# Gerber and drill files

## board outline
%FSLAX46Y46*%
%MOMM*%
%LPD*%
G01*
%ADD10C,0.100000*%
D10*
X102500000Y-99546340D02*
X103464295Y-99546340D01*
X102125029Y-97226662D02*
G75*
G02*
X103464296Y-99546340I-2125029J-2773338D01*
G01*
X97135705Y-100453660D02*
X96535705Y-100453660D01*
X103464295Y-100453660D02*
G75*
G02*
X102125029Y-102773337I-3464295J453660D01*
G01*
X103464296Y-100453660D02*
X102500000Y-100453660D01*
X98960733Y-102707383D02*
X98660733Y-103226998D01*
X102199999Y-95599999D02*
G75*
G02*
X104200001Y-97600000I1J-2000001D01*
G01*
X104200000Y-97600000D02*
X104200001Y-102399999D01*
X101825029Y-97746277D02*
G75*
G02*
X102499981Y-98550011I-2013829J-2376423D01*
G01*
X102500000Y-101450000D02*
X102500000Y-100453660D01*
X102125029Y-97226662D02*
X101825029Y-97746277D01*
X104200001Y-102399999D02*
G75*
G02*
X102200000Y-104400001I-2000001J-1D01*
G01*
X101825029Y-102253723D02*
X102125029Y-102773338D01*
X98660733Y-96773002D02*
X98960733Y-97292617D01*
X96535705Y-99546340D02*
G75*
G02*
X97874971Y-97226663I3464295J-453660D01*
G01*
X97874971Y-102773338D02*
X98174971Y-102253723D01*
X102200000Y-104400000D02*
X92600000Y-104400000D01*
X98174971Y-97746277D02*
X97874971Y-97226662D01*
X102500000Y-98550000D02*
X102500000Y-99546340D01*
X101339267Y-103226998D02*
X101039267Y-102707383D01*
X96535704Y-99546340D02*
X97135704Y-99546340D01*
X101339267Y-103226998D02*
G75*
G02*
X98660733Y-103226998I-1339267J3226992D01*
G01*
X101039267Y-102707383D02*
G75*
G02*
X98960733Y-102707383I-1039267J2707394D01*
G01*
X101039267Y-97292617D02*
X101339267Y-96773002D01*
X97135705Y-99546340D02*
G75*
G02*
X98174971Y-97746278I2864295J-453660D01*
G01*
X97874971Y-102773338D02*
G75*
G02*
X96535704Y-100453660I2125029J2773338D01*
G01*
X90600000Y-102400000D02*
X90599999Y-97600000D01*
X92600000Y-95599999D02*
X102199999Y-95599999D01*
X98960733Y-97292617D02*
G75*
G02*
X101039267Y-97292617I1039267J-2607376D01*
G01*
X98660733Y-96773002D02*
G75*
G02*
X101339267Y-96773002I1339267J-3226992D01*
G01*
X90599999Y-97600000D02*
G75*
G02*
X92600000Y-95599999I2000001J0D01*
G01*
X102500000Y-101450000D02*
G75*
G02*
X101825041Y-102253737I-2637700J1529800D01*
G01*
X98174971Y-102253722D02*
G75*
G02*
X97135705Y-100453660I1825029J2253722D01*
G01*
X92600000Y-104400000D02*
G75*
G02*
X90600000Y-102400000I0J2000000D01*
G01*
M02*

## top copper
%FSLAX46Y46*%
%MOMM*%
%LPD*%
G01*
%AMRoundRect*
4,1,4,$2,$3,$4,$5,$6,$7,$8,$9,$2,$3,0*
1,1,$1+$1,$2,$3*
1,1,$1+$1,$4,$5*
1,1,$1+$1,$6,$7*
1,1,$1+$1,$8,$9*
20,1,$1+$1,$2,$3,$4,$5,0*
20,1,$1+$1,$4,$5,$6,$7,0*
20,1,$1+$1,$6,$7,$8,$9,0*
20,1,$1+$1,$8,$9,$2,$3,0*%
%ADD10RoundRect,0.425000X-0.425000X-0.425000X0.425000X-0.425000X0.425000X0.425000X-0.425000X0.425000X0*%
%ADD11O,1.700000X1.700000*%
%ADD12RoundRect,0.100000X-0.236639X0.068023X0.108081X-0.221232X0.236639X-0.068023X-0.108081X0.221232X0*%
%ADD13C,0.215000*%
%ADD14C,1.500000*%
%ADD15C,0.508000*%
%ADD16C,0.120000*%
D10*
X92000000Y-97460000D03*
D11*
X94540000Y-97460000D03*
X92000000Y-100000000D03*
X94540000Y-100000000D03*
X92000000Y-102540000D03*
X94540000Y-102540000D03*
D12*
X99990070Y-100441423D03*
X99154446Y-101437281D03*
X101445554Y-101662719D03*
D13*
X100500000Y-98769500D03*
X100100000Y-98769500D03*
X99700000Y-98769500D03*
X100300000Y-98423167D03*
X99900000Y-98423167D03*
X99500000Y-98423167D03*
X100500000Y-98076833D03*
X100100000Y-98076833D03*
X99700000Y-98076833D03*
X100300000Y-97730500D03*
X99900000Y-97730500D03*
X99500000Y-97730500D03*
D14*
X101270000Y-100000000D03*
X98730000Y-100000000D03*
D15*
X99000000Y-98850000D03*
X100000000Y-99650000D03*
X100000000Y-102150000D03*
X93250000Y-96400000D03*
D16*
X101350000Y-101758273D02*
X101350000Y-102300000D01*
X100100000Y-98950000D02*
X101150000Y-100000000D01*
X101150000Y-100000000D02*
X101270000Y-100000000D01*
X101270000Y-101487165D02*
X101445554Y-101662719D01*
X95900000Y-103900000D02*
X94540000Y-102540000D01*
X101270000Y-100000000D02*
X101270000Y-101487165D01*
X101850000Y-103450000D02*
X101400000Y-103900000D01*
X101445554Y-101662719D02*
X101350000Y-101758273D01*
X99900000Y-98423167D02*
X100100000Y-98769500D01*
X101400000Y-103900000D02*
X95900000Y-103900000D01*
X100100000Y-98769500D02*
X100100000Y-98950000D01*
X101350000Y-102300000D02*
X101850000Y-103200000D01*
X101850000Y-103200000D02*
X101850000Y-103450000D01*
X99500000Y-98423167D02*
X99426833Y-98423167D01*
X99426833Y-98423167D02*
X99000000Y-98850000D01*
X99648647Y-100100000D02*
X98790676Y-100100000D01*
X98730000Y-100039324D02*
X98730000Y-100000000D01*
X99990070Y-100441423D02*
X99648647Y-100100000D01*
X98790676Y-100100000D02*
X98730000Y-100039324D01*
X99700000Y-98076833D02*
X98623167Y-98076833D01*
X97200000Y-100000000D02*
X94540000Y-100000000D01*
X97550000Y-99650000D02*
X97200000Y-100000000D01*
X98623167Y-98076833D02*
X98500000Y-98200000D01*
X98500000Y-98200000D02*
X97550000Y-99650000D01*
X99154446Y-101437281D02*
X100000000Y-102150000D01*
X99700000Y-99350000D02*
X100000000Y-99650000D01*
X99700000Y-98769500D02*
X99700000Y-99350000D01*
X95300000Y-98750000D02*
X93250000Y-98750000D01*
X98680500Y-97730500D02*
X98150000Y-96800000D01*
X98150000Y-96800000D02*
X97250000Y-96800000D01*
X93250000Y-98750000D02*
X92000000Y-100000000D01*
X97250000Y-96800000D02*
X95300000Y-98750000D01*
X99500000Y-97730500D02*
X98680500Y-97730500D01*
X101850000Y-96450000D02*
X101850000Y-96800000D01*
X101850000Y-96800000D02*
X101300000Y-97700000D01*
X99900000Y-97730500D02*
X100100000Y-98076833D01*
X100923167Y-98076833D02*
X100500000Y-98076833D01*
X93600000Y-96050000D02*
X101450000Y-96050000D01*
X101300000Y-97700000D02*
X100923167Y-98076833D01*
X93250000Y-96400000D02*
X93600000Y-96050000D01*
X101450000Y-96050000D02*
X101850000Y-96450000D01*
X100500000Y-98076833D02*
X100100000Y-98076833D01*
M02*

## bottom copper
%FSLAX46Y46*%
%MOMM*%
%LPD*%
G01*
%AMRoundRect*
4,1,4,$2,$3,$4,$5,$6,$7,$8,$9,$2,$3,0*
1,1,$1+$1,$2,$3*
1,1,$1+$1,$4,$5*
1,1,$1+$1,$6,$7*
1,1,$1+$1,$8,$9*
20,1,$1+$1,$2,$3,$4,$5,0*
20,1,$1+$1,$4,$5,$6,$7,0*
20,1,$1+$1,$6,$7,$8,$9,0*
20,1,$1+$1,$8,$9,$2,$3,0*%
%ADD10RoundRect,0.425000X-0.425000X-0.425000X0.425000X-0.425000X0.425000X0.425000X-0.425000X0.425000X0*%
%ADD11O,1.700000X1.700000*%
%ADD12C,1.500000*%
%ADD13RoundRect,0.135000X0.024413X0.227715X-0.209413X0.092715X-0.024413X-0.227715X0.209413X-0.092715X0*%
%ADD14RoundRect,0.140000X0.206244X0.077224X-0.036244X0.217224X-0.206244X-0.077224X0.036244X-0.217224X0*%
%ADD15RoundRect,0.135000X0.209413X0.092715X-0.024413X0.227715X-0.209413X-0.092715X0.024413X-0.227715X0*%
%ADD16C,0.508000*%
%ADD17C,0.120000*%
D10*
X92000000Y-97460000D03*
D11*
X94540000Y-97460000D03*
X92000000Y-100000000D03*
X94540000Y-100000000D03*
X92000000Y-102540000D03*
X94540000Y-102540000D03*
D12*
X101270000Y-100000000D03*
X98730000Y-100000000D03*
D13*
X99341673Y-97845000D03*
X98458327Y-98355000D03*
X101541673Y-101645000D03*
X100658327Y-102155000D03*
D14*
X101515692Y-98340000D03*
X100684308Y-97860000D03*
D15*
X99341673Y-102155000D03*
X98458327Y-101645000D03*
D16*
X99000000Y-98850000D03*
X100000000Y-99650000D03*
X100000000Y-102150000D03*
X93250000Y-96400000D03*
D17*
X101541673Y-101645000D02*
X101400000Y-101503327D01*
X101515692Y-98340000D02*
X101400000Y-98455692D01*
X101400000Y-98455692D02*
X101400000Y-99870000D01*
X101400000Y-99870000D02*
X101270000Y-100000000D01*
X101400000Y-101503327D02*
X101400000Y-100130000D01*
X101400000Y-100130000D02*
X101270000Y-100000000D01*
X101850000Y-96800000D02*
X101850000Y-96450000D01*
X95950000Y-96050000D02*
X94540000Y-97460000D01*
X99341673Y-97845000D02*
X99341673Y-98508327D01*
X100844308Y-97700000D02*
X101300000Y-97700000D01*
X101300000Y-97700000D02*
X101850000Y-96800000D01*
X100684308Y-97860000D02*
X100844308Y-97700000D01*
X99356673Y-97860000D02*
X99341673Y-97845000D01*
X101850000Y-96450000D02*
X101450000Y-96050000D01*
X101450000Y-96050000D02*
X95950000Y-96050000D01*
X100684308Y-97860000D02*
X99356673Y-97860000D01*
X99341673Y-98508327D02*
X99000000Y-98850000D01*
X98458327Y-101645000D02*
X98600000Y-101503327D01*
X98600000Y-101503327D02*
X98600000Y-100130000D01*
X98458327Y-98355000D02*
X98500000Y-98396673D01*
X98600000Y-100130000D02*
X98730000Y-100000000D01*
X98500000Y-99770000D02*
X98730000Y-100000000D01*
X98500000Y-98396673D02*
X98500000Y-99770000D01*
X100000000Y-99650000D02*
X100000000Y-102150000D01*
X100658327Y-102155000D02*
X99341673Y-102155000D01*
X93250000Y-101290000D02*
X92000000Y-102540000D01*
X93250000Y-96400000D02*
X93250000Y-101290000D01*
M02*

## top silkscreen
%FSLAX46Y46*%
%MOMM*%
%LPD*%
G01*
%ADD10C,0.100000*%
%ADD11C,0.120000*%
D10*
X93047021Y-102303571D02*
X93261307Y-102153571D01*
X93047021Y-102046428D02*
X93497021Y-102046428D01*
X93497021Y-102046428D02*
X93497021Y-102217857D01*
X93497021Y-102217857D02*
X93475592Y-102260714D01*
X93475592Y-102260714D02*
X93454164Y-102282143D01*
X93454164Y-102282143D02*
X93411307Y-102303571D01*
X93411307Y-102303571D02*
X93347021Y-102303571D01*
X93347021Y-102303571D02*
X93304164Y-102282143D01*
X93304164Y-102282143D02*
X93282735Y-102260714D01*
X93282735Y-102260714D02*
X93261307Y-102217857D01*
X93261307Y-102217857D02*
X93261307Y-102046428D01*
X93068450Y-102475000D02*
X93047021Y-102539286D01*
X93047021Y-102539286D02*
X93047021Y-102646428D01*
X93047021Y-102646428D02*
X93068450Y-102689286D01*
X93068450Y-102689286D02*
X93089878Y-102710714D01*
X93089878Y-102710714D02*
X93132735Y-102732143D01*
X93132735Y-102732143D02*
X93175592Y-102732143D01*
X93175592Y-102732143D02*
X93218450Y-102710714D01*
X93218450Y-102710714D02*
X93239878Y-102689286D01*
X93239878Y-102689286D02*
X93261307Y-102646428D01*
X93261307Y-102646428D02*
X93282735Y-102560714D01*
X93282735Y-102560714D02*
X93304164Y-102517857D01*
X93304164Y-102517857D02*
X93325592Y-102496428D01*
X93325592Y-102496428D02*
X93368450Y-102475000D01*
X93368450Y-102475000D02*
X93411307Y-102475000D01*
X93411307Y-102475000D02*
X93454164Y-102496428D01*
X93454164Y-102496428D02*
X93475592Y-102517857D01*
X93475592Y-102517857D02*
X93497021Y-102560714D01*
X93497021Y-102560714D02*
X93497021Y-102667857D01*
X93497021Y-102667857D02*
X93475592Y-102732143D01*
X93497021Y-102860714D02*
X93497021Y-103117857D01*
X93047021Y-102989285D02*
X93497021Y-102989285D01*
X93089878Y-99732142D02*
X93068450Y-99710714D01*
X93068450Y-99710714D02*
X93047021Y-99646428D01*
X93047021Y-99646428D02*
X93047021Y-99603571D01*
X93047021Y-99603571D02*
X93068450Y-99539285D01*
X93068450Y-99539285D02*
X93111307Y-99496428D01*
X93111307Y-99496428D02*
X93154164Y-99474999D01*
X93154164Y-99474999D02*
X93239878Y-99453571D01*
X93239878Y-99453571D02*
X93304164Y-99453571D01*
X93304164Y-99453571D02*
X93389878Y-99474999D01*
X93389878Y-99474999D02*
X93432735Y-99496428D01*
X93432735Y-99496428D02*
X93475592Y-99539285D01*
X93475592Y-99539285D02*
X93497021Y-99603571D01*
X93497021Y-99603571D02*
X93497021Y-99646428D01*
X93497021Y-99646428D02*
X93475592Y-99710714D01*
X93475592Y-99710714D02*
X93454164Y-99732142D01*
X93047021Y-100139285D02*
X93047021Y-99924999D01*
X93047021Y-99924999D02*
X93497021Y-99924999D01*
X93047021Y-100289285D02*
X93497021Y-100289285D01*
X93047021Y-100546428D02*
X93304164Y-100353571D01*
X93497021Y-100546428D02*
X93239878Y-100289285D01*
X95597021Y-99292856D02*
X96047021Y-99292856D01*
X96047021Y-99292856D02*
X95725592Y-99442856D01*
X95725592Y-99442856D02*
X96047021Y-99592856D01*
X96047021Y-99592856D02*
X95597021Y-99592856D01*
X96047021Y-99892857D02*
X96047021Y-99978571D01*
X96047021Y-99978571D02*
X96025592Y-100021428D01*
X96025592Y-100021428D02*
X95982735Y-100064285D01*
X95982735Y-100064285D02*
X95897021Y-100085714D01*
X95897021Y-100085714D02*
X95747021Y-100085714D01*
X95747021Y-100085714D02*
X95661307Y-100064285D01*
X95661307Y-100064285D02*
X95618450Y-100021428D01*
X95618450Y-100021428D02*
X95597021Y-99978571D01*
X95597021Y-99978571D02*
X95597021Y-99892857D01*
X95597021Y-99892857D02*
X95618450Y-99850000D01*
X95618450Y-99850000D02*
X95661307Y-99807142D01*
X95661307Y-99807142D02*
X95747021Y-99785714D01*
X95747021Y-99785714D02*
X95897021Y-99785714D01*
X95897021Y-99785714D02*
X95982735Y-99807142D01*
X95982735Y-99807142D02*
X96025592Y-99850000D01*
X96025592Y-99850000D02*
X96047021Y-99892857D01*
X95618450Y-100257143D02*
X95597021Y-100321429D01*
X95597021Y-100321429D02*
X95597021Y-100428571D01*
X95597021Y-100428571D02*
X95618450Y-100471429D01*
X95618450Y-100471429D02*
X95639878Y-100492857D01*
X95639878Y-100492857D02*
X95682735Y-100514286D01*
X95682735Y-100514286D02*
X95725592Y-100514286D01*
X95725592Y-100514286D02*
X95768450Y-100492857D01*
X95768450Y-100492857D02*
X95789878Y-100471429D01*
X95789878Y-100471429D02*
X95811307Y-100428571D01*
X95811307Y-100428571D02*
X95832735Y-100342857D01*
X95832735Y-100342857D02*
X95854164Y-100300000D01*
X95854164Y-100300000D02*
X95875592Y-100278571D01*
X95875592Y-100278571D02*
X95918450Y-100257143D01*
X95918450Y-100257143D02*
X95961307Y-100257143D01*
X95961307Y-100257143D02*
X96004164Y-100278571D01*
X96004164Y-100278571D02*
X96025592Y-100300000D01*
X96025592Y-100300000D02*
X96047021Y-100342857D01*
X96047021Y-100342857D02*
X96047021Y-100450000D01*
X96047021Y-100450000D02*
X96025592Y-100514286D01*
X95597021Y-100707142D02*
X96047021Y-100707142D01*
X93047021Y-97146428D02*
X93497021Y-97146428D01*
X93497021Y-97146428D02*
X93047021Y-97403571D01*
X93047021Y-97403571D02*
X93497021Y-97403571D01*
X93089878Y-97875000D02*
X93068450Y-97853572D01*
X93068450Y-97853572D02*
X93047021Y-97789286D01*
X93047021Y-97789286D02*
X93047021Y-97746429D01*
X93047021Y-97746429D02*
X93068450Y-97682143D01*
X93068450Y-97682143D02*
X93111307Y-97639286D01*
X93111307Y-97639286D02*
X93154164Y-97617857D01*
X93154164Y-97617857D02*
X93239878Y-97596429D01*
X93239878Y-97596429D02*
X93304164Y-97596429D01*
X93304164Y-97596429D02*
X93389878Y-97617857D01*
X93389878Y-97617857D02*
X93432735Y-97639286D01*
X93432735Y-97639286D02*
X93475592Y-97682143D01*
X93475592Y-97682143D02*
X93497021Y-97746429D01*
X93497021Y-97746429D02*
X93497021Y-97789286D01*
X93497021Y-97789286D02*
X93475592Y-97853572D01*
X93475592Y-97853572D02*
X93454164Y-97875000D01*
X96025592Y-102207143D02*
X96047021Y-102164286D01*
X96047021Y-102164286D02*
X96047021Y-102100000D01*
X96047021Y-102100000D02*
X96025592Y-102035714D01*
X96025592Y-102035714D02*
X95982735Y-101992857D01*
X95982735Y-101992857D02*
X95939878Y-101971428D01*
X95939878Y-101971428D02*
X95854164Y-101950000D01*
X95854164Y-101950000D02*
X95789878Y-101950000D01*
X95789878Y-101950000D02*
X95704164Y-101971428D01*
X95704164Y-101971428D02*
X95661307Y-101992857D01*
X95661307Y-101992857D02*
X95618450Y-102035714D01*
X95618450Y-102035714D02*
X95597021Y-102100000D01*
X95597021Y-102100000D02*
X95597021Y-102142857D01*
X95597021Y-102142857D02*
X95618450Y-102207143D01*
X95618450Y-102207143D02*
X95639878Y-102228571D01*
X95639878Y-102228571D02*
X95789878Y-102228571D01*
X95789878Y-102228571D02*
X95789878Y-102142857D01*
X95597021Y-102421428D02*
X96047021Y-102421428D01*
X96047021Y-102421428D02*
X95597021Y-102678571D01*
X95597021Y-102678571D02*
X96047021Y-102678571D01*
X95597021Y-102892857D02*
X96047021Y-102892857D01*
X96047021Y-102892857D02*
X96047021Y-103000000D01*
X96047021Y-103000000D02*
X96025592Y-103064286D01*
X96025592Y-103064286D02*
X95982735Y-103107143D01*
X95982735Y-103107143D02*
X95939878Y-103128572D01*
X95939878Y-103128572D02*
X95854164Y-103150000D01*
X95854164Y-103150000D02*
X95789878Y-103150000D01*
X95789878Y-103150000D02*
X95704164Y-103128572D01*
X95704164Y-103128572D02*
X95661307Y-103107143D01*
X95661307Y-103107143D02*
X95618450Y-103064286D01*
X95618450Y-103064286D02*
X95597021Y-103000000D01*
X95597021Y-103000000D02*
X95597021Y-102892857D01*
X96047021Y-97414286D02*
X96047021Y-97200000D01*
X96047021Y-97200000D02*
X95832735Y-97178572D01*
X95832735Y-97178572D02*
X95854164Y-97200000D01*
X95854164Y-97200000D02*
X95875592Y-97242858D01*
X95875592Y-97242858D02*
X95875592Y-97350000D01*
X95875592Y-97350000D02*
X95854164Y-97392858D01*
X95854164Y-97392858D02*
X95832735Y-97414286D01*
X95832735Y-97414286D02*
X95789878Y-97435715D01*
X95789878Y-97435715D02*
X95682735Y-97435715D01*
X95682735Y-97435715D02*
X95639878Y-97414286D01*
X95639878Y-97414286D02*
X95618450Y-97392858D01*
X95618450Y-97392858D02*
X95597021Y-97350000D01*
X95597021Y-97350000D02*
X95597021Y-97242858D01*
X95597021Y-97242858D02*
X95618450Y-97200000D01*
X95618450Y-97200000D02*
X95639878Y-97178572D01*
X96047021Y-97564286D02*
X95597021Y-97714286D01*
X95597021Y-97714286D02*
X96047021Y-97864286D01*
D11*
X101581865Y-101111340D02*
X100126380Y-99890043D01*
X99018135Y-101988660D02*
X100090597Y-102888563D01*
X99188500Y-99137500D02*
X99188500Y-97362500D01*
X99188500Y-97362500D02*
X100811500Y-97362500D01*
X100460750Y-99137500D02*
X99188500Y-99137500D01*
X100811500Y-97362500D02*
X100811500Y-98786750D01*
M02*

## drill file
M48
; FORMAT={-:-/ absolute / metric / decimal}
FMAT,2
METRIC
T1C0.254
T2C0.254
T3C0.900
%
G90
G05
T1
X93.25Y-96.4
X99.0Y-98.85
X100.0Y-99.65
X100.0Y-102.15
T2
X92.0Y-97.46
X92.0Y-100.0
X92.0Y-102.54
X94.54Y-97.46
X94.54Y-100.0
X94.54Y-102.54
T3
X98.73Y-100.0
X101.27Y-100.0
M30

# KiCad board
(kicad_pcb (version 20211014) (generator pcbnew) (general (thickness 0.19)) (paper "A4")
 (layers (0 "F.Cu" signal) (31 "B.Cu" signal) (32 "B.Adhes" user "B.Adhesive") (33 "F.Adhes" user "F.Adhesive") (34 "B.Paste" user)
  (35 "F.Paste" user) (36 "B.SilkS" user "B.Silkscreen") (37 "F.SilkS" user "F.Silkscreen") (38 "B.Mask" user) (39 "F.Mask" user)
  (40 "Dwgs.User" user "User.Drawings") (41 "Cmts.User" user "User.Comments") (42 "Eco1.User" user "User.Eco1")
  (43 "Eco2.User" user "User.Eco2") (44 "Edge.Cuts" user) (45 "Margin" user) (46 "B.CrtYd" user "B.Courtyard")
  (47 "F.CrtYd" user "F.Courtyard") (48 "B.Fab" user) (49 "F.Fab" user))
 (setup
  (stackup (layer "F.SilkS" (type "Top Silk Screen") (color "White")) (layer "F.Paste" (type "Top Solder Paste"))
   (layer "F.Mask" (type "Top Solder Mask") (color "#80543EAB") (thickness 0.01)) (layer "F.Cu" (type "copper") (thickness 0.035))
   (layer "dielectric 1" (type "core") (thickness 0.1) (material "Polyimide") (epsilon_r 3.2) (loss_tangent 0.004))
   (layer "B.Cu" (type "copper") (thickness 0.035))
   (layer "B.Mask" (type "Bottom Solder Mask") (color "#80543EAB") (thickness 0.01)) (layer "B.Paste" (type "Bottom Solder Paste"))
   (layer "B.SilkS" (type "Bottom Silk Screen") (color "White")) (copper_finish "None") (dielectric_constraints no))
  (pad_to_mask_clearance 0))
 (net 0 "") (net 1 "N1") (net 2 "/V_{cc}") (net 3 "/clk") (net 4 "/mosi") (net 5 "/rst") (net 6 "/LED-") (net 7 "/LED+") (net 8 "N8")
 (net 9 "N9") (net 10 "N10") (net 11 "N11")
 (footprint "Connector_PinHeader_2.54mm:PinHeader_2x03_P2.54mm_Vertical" (layer "F.Cu") (at 92 97.46)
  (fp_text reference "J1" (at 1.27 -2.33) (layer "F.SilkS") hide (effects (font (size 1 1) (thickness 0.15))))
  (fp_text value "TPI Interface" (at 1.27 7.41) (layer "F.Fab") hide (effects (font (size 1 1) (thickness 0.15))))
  (pad "1" thru_hole roundrect (at 0 0) (size 1.7 1.7) (drill 0.254) (layers *.Cu *.Mask) (roundrect_rratio 0.25) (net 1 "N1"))
  (pad "2" thru_hole oval (at 2.54 0) (size 1.7 1.7) (drill 0.254) (layers *.Cu *.Mask) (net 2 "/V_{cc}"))
  (pad "3" thru_hole oval (at 0 2.54) (size 1.7 1.7) (drill 0.254) (layers *.Cu *.Mask) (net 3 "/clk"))
  (pad "4" thru_hole oval (at 2.54 2.54) (size 1.7 1.7) (drill 0.254) (layers *.Cu *.Mask) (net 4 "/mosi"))
  (pad "5" thru_hole oval (at 0 5.08) (size 1.7 1.7) (drill 0.254) (layers *.Cu *.Mask) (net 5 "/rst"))
  (pad "6" thru_hole oval (at 2.54 5.08) (size 1.7 1.7) (drill 0.254) (layers *.Cu *.Mask) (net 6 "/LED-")))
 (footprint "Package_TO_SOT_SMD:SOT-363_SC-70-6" (layer "F.Cu") (at 100.3 101.55 -40)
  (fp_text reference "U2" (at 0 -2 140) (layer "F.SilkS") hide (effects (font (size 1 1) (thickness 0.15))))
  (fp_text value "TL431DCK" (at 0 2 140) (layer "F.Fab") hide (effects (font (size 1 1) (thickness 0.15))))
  (fp_line (start 0.7 -1.16) (end -1.2 -1.16) (layer "F.SilkS") (width 0.12))
  (fp_line (start -0.7 1.16) (end 0.7 1.16) (layer "F.SilkS") (width 0.12))
  (pad "1" smd roundrect (at -0.95 -0.65 320) (size 0.65 0.4) (layers "F.Cu" "F.Paste" "F.Mask") (roundrect_rratio 0.25) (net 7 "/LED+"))
  (pad "3" smd roundrect (at -0.95 0.65 320) (size 0.65 0.4) (layers "F.Cu" "F.Paste" "F.Mask") (roundrect_rratio 0.25) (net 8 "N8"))
  (pad "6" smd roundrect (at 0.95 -0.65 320) (size 0.65 0.4) (layers "F.Cu" "F.Paste" "F.Mask") (roundrect_rratio 0.25) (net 6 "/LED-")))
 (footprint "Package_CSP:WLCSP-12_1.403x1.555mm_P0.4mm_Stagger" (layer "F.Cu") (at 100 98.25 180) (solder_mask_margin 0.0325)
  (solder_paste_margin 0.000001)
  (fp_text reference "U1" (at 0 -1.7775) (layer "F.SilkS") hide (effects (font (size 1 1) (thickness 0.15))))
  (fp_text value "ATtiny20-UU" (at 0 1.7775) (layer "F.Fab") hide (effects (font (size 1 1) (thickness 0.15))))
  (fp_line (start 0.8115 -0.8875) (end 0.8115 0.8875) (layer "F.SilkS") (width 0.12))
  (fp_line (start 0.8115 0.8875) (end -0.8115 0.8875) (layer "F.SilkS") (width 0.12))
  (fp_line (start -0.46075 -0.8875) (end 0.8115 -0.8875) (layer "F.SilkS") (width 0.12))
  (fp_line (start -0.8115 0.8875) (end -0.8115 -0.53675) (layer "F.SilkS") (width 0.12))
  (pad "A1" smd circle locked (at -0.5 -0.5195 180) (size 0.215 0.215) (layers "F.Cu" "F.Paste" "F.Mask") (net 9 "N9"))
  (pad "A3" smd circle locked (at -0.1 -0.5195 180) (size 0.215 0.215) (layers "F.Cu" "F.Paste" "F.Mask") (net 6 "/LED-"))
  (pad "A5" smd circle locked (at 0.3 -0.5195 180) (size 0.215 0.215) (layers "F.Cu" "F.Paste" "F.Mask") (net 8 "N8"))
  (pad "B2" smd circle locked (at -0.3 -0.173167 180) (size 0.215 0.215) (layers "F.Cu" "F.Paste" "F.Mask") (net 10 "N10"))
  (pad "B4" smd circle locked (at 0.1 -0.173167 180) (size 0.215 0.215) (layers "F.Cu" "F.Paste" "F.Mask") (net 6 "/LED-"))
  (pad "B6" smd circle locked (at 0.5 -0.173167 180) (size 0.215 0.215) (layers "F.Cu" "F.Paste" "F.Mask") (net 2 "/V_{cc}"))
  (pad "C1" smd circle locked (at -0.5 0.173167 180) (size 0.215 0.215) (layers "F.Cu" "F.Paste" "F.Mask") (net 5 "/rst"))
  (pad "C3" smd circle locked (at -0.1 0.173167 180) (size 0.215 0.215) (layers "F.Cu" "F.Paste" "F.Mask") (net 5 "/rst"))
  (pad "C5" smd circle locked (at 0.3 0.173167 180) (size 0.215 0.215) (layers "F.Cu" "F.Paste" "F.Mask") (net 4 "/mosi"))
  (pad "D2" smd circle locked (at -0.3 0.5195 180) (size 0.215 0.215) (layers "F.Cu" "F.Paste" "F.Mask") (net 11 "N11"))
  (pad "D4" smd circle locked (at 0.1 0.5195 180) (size 0.215 0.215) (layers "F.Cu" "F.Paste" "F.Mask") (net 5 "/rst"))
  (pad "D6" smd circle locked (at 0.5 0.5195 180) (size 0.215 0.215) (layers "F.Cu" "F.Paste" "F.Mask") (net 3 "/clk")))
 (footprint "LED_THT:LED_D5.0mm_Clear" (layer "B.Cu") (at 100 100 180)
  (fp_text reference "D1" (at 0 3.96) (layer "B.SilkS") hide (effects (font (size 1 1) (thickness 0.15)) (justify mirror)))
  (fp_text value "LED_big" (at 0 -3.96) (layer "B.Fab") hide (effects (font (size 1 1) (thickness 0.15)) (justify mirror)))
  (pad "1" thru_hole circle (at -1.27 0 180) (size 1.5 1.5) (drill 0.9) (layers *.Cu *.Mask) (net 6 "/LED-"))
  (pad "2" thru_hole circle (at 1.27 0 180) (size 1.5 1.5) (drill 0.9) (layers *.Cu *.Mask) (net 7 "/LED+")))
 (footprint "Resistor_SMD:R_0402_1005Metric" (layer "B.Cu") (at 98.9 98.1 -150)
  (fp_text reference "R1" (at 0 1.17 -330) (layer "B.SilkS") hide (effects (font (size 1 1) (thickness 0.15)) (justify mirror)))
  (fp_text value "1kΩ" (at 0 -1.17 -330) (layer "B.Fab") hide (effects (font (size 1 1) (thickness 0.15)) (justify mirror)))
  (pad "1" smd roundrect locked (at -0.51 0 210) (size 0.54 0.64) (layers "B.Cu" "B.Paste" "B.Mask") (roundrect_rratio 0.25)
   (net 2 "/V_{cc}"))
  (pad "2" smd roundrect locked (at 0.51 0 210) (size 0.54 0.64) (layers "B.Cu" "B.Paste" "B.Mask") (roundrect_rratio 0.25) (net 7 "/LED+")))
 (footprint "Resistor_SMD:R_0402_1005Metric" (layer "B.Cu") (at 101.1 101.9 -150)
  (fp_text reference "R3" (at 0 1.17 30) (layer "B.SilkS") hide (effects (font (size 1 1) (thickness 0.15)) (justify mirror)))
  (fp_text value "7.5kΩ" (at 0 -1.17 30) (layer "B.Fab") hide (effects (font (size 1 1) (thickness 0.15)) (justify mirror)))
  (pad "1" smd roundrect locked (at -0.51 0 210) (size 0.54 0.64) (layers "B.Cu" "B.Paste" "B.Mask") (roundrect_rratio 0.25) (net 6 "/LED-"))
  (pad "2" smd roundrect locked (at 0.51 0 210) (size 0.54 0.64) (layers "B.Cu" "B.Paste" "B.Mask") (roundrect_rratio 0.25) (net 8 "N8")))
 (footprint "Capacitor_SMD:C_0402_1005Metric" (layer "B.Cu") (at 101.1 98.1 150)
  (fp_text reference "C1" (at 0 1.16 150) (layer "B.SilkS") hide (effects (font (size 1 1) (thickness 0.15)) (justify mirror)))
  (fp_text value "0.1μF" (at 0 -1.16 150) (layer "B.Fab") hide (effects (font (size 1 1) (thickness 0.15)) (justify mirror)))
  (pad "1" smd roundrect locked (at -0.48 0 150) (size 0.56 0.62) (layers "B.Cu" "B.Paste" "B.Mask") (roundrect_rratio 0.25) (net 6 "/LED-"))
  (pad "2" smd roundrect locked (at 0.48 0 150) (size 0.56 0.62) (layers "B.Cu" "B.Paste" "B.Mask") (roundrect_rratio 0.25)
   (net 2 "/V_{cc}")))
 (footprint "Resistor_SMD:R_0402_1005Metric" (layer "B.Cu") (at 98.9 101.9 150)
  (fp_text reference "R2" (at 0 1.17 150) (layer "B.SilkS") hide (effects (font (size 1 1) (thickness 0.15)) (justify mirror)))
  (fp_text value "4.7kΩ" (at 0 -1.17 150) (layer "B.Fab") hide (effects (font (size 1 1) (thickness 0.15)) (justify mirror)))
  (pad "1" smd roundrect locked (at -0.51 0 150) (size 0.54 0.64) (layers "B.Cu" "B.Paste" "B.Mask") (roundrect_rratio 0.25) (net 8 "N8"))
  (pad "2" smd roundrect locked (at 0.51 0 150) (size 0.54 0.64) (layers "B.Cu" "B.Paste" "B.Mask") (roundrect_rratio 0.25) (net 7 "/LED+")))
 (gr_line (start 102.5 99.54634) (end 103.464295 99.54634) (layer "Edge.Cuts") (width 0.1))
 (gr_arc (start 102.125029 97.226662) (mid 103.025783 98.253063) (end 103.464295 99.54634) (layer "Edge.Cuts") (width 0.1))
 (gr_line (start 97.135705 100.45366) (end 96.535705 100.45366) (layer "Edge.Cuts") (width 0.1))
 (gr_arc (start 103.464295 100.45366) (mid 103.025783 101.746936) (end 102.125029 102.773338) (layer "Edge.Cuts") (width 0.1))
 (gr_line (start 103.464296 100.45366) (end 102.5 100.45366) (layer "Edge.Cuts") (width 0.1))
 (gr_line (start 98.960733 102.707383) (end 98.660733 103.226998) (layer "Edge.Cuts") (width 0.1))
 (gr_arc (start 102.199999 95.599999) (mid 103.614213 96.185786) (end 104.2 97.6) (layer "Edge.Cuts") (width 0.1))
 (gr_line (start 104.2 97.6) (end 104.200001 102.399999) (layer "Edge.Cuts") (width 0.1))
 (gr_arc (start 101.825029 97.746277) (mid 102.196609 98.119506) (end 102.5 98.55) (layer "Edge.Cuts") (width 0.1))
 (gr_line (start 102.5 101.45) (end 102.5 100.45366) (layer "Edge.Cuts") (width 0.1))
 (gr_line (start 102.125029 97.226662) (end 101.825029 97.746277) (layer "Edge.Cuts") (width 0.1))
 (gr_arc (start 104.200001 102.399999) (mid 103.614214 103.814213) (end 102.2 104.4) (layer "Edge.Cuts") (width 0.1))
 (gr_line (start 101.825029 102.253723) (end 102.125029 102.773338) (layer "Edge.Cuts") (width 0.1))
 (gr_line (start 98.660733 96.773002) (end 98.960733 97.292617) (layer "Edge.Cuts") (width 0.1))
 (gr_arc (start 96.535705 99.54634) (mid 96.974217 98.253064) (end 97.874971 97.226662) (layer "Edge.Cuts") (width 0.1))
 (gr_line (start 97.874971 102.773338) (end 98.174971 102.253723) (layer "Edge.Cuts") (width 0.1))
 (gr_line (start 102.2 104.4) (end 92.6 104.4) (layer "Edge.Cuts") (width 0.1))
 (gr_line (start 98.174971 97.746277) (end 97.874971 97.226662) (layer "Edge.Cuts") (width 0.1))
 (gr_line (start 102.5 98.55) (end 102.5 99.54634) (layer "Edge.Cuts") (width 0.1))
 (gr_line (start 101.339267 103.226998) (end 101.039267 102.707383) (layer "Edge.Cuts") (width 0.1))
 (gr_line (start 96.535704 99.54634) (end 97.135704 99.54634) (layer "Edge.Cuts") (width 0.1))
 (gr_arc (start 101.339267 103.226998) (mid 100 103.493874) (end 98.660733 103.226998) (layer "Edge.Cuts") (width 0.1))
 (gr_arc (start 101.039267 102.707383) (mid 100 102.899999) (end 98.960733 102.707383) (layer "Edge.Cuts") (width 0.1))
 (gr_line (start 101.039267 97.292617) (end 101.339267 96.773002) (layer "Edge.Cuts") (width 0.1))
 (gr_arc (start 97.135705 99.54634) (mid 97.488527 98.550001) (end 98.174971 97.746278) (layer "Edge.Cuts") (width 0.1))
 (gr_arc (start 97.874971 102.773338) (mid 96.974217 101.746937) (end 96.535705 100.45366) (layer "Edge.Cuts") (width 0.1))
 (gr_line (start 90.6 102.4) (end 90.599999 97.6) (layer "Edge.Cuts") (width 0.1))
 (gr_line (start 92.6 95.599999) (end 102.199999 95.599999) (layer "Edge.Cuts") (width 0.1))
 (gr_arc (start 98.960733 97.292617) (mid 100 97.093129) (end 101.039267 97.292617) (layer "Edge.Cuts") (width 0.1))
 (gr_arc (start 98.660733 96.773002) (mid 100 96.506126) (end 101.339267 96.773002) (layer "Edge.Cuts") (width 0.1))
 (gr_arc (start 90.599999 97.6) (mid 91.185786 96.185786) (end 92.6 95.599999) (layer "Edge.Cuts") (width 0.1))
 (gr_arc (start 102.5 101.45) (mid 102.197355 101.881121) (end 101.825029 102.253723) (layer "Edge.Cuts") (width 0.1))
 (gr_arc (start 98.174971 102.253722) (mid 97.488527 101.449999) (end 97.135705 100.45366) (layer "Edge.Cuts") (width 0.1))
 (gr_arc (start 92.6 104.4) (mid 91.185786 103.814214) (end 90.6 102.4) (layer "Edge.Cuts") (width 0.1))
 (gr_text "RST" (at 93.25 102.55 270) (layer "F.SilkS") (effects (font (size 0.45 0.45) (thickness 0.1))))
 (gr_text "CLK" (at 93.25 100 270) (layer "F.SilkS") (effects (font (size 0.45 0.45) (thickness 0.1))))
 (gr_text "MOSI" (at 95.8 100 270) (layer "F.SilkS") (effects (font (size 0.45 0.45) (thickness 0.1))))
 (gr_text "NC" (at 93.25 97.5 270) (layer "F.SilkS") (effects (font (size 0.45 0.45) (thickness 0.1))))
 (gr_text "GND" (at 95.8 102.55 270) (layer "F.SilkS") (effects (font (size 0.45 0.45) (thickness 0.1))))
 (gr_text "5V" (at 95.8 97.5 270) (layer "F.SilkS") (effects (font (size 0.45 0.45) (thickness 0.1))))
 (segment (start 101.35 101.758273) (end 101.35 102.3) (width 0.12) (layer "F.Cu") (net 6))
 (segment (start 100.1 98.95) (end 101.15 100) (width 0.12) (layer "F.Cu") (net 6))
 (segment (start 101.15 100) (end 101.27 100) (width 0.12) (layer "F.Cu") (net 6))
 (segment (start 101.27 101.487165) (end 101.445554 101.662719) (width 0.12) (layer "F.Cu") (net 6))
 (segment (start 95.9 103.9) (end 94.54 102.54) (width 0.12) (layer "F.Cu") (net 6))
 (segment (start 101.27 100) (end 101.27 101.487165) (width 0.12) (layer "F.Cu") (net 6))
 (segment (start 101.85 103.45) (end 101.4 103.9) (width 0.12) (layer "F.Cu") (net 6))
 (segment (start 101.445554 101.662719) (end 101.35 101.758273) (width 0.12) (layer "F.Cu") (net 6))
 (segment (start 99.9 98.423167) (end 100.1 98.7695) (width 0.12) (layer "F.Cu") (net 6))
 (segment (start 101.4 103.9) (end 95.9 103.9) (width 0.12) (layer "F.Cu") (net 6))
 (segment (start 100.1 98.7695) (end 100.1 98.95) (width 0.12) (layer "F.Cu") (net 6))
 (segment (start 101.35 102.3) (end 101.85 103.2) (width 0.12) (layer "F.Cu") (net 6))
 (segment (start 101.85 103.2) (end 101.85 103.45) (width 0.12) (layer "F.Cu") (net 6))
 (segment (start 101.541673 101.645) (end 101.4 101.503327) (width 0.12) (layer "B.Cu") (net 6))
 (segment (start 101.515692 98.34) (end 101.4 98.455692) (width 0.12) (layer "B.Cu") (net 6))
 (segment (start 101.4 98.455692) (end 101.4 99.87) (width 0.12) (layer "B.Cu") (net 6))
 (segment (start 101.4 99.87) (end 101.27 100) (width 0.12) (layer "B.Cu") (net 6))
 (segment (start 101.4 101.503327) (end 101.4 100.13) (width 0.12) (layer "B.Cu") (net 6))
 (segment (start 101.4 100.13) (end 101.27 100) (width 0.12) (layer "B.Cu") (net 6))
 (segment (start 99.5 98.423167) (end 99.426833 98.423167) (width 0.12) (layer "F.Cu") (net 2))
 (segment (start 99.426833 98.423167) (end 99 98.85) (width 0.12) (layer "F.Cu") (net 2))
 (via (at 99 98.85) (size 0.508) (drill 0.254) (layers "F.Cu" "B.Cu") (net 2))
 (segment (start 101.85 96.8) (end 101.85 96.45) (width 0.12) (layer "B.Cu") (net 2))
 (segment (start 95.95 96.05) (end 94.54 97.46) (width 0.12) (layer "B.Cu") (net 2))
 (segment (start 99.341673 97.845) (end 99.341673 98.508327) (width 0.12) (layer "B.Cu") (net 2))
 (segment (start 100.844308 97.7) (end 101.3 97.7) (width 0.12) (layer "B.Cu") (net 2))
 (segment (start 101.3 97.7) (end 101.85 96.8) (width 0.12) (layer "B.Cu") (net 2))
 (segment (start 100.684308 97.86) (end 100.844308 97.7) (width 0.12) (layer "B.Cu") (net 2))
 (segment (start 99.356673 97.86) (end 99.341673 97.845) (width 0.12) (layer "B.Cu") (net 2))
 (segment (start 101.85 96.45) (end 101.45 96.05) (width 0.12) (layer "B.Cu") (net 2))
 (segment (start 101.45 96.05) (end 95.95 96.05) (width 0.12) (layer "B.Cu") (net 2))
 (segment (start 100.684308 97.86) (end 99.356673 97.86) (width 0.12) (layer "B.Cu") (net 2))
 (segment (start 99.341673 98.508327) (end 99 98.85) (width 0.12) (layer "B.Cu") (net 2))
 (segment (start 99.648647 100.1) (end 98.790676 100.1) (width 0.12) (layer "F.Cu") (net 7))
 (segment (start 98.73 100.039324) (end 98.73 100) (width 0.12) (layer "F.Cu") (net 7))
 (segment (start 99.99007 100.441423) (end 99.648647 100.1) (width 0.12) (layer "F.Cu") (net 7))
 (segment (start 98.790676 100.1) (end 98.73 100.039324) (width 0.12) (layer "F.Cu") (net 7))
 (segment (start 98.458327 101.645) (end 98.6 101.503327) (width 0.12) (layer "B.Cu") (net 7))
 (segment (start 98.6 101.503327) (end 98.6 100.13) (width 0.12) (layer "B.Cu") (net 7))
 (segment (start 98.458327 98.355) (end 98.5 98.396673) (width 0.12) (layer "B.Cu") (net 7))
 (segment (start 98.6 100.13) (end 98.73 100) (width 0.12) (layer "B.Cu") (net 7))
 (segment (start 98.5 99.77) (end 98.73 100) (width 0.12) (layer "B.Cu") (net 7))
 (segment (start 98.5 98.396673) (end 98.5 99.77) (width 0.12) (layer "B.Cu") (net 7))
 (segment (start 99.7 98.076833) (end 98.623167 98.076833) (width 0.12) (layer "F.Cu") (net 4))
 (segment (start 97.2 100) (end 94.54 100) (width 0.12) (layer "F.Cu") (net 4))
 (segment (start 97.55 99.65) (end 97.2 100) (width 0.12) (layer "F.Cu") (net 4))
 (segment (start 98.623167 98.076833) (end 98.5 98.2) (width 0.12) (layer "F.Cu") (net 4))
 (segment (start 98.5 98.2) (end 97.55 99.65) (width 0.12) (layer "F.Cu") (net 4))
 (segment (start 99.154446 101.437281) (end 100 102.15) (width 0.12) (layer "F.Cu") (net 8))
 (segment (start 99.7 99.35) (end 100 99.65) (width 0.12) (layer "F.Cu") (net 8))
 (segment (start 99.7 98.7695) (end 99.7 99.35) (width 0.12) (layer "F.Cu") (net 8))
 (via (at 100 99.65) (size 0.508) (drill 0.254) (layers "F.Cu" "B.Cu") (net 8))
 (via (at 100 102.15) (size 0.508) (drill 0.254) (layers "F.Cu" "B.Cu") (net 8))
 (segment (start 100 99.65) (end 100 102.15) (width 0.12) (layer "B.Cu") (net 8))
 (segment (start 100.658327 102.155) (end 99.341673 102.155) (width 0.12) (layer "B.Cu") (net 8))
 (segment (start 95.3 98.75) (end 93.25 98.75) (width 0.12) (layer "F.Cu") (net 3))
 (segment (start 98.6805 97.7305) (end 98.15 96.8) (width 0.12) (layer "F.Cu") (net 3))
 (segment (start 98.15 96.8) (end 97.25 96.8) (width 0.12) (layer "F.Cu") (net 3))
 (segment (start 93.25 98.75) (end 92 100) (width 0.12) (layer "F.Cu") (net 3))
 (segment (start 97.25 96.8) (end 95.3 98.75) (width 0.12) (layer "F.Cu") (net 3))
 (segment (start 99.5 97.7305) (end 98.6805 97.7305) (width 0.12) (layer "F.Cu") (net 3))
 (segment (start 101.85 96.45) (end 101.85 96.8) (width 0.12) (layer "F.Cu") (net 5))
 (segment (start 101.85 96.8) (end 101.3 97.7) (width 0.12) (layer "F.Cu") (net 5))
 (segment (start 99.9 97.7305) (end 100.1 98.076833) (width 0.12) (layer "F.Cu") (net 5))
 (segment (start 100.923167 98.076833) (end 100.5 98.076833) (width 0.12) (layer "F.Cu") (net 5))
 (segment (start 93.6 96.05) (end 101.45 96.05) (width 0.12) (layer "F.Cu") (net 5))
 (segment (start 101.3 97.7) (end 100.923167 98.076833) (width 0.12) (layer "F.Cu") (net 5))
 (segment (start 93.25 96.4) (end 93.6 96.05) (width 0.12) (layer "F.Cu") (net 5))
 (segment (start 101.45 96.05) (end 101.85 96.45) (width 0.12) (layer "F.Cu") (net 5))
 (segment (start 100.5 98.076833) (end 100.1 98.076833) (width 0.12) (layer "F.Cu") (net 5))
 (via (at 93.25 96.4) (size 0.508) (drill 0.254) (layers "F.Cu" "B.Cu") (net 5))
 (segment (start 93.25 101.29) (end 92 102.54) (width 0.12) (layer "B.Cu") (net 5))
 (segment (start 93.25 96.4) (end 93.25 101.29) (width 0.12) (layer "B.Cu") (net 5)))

